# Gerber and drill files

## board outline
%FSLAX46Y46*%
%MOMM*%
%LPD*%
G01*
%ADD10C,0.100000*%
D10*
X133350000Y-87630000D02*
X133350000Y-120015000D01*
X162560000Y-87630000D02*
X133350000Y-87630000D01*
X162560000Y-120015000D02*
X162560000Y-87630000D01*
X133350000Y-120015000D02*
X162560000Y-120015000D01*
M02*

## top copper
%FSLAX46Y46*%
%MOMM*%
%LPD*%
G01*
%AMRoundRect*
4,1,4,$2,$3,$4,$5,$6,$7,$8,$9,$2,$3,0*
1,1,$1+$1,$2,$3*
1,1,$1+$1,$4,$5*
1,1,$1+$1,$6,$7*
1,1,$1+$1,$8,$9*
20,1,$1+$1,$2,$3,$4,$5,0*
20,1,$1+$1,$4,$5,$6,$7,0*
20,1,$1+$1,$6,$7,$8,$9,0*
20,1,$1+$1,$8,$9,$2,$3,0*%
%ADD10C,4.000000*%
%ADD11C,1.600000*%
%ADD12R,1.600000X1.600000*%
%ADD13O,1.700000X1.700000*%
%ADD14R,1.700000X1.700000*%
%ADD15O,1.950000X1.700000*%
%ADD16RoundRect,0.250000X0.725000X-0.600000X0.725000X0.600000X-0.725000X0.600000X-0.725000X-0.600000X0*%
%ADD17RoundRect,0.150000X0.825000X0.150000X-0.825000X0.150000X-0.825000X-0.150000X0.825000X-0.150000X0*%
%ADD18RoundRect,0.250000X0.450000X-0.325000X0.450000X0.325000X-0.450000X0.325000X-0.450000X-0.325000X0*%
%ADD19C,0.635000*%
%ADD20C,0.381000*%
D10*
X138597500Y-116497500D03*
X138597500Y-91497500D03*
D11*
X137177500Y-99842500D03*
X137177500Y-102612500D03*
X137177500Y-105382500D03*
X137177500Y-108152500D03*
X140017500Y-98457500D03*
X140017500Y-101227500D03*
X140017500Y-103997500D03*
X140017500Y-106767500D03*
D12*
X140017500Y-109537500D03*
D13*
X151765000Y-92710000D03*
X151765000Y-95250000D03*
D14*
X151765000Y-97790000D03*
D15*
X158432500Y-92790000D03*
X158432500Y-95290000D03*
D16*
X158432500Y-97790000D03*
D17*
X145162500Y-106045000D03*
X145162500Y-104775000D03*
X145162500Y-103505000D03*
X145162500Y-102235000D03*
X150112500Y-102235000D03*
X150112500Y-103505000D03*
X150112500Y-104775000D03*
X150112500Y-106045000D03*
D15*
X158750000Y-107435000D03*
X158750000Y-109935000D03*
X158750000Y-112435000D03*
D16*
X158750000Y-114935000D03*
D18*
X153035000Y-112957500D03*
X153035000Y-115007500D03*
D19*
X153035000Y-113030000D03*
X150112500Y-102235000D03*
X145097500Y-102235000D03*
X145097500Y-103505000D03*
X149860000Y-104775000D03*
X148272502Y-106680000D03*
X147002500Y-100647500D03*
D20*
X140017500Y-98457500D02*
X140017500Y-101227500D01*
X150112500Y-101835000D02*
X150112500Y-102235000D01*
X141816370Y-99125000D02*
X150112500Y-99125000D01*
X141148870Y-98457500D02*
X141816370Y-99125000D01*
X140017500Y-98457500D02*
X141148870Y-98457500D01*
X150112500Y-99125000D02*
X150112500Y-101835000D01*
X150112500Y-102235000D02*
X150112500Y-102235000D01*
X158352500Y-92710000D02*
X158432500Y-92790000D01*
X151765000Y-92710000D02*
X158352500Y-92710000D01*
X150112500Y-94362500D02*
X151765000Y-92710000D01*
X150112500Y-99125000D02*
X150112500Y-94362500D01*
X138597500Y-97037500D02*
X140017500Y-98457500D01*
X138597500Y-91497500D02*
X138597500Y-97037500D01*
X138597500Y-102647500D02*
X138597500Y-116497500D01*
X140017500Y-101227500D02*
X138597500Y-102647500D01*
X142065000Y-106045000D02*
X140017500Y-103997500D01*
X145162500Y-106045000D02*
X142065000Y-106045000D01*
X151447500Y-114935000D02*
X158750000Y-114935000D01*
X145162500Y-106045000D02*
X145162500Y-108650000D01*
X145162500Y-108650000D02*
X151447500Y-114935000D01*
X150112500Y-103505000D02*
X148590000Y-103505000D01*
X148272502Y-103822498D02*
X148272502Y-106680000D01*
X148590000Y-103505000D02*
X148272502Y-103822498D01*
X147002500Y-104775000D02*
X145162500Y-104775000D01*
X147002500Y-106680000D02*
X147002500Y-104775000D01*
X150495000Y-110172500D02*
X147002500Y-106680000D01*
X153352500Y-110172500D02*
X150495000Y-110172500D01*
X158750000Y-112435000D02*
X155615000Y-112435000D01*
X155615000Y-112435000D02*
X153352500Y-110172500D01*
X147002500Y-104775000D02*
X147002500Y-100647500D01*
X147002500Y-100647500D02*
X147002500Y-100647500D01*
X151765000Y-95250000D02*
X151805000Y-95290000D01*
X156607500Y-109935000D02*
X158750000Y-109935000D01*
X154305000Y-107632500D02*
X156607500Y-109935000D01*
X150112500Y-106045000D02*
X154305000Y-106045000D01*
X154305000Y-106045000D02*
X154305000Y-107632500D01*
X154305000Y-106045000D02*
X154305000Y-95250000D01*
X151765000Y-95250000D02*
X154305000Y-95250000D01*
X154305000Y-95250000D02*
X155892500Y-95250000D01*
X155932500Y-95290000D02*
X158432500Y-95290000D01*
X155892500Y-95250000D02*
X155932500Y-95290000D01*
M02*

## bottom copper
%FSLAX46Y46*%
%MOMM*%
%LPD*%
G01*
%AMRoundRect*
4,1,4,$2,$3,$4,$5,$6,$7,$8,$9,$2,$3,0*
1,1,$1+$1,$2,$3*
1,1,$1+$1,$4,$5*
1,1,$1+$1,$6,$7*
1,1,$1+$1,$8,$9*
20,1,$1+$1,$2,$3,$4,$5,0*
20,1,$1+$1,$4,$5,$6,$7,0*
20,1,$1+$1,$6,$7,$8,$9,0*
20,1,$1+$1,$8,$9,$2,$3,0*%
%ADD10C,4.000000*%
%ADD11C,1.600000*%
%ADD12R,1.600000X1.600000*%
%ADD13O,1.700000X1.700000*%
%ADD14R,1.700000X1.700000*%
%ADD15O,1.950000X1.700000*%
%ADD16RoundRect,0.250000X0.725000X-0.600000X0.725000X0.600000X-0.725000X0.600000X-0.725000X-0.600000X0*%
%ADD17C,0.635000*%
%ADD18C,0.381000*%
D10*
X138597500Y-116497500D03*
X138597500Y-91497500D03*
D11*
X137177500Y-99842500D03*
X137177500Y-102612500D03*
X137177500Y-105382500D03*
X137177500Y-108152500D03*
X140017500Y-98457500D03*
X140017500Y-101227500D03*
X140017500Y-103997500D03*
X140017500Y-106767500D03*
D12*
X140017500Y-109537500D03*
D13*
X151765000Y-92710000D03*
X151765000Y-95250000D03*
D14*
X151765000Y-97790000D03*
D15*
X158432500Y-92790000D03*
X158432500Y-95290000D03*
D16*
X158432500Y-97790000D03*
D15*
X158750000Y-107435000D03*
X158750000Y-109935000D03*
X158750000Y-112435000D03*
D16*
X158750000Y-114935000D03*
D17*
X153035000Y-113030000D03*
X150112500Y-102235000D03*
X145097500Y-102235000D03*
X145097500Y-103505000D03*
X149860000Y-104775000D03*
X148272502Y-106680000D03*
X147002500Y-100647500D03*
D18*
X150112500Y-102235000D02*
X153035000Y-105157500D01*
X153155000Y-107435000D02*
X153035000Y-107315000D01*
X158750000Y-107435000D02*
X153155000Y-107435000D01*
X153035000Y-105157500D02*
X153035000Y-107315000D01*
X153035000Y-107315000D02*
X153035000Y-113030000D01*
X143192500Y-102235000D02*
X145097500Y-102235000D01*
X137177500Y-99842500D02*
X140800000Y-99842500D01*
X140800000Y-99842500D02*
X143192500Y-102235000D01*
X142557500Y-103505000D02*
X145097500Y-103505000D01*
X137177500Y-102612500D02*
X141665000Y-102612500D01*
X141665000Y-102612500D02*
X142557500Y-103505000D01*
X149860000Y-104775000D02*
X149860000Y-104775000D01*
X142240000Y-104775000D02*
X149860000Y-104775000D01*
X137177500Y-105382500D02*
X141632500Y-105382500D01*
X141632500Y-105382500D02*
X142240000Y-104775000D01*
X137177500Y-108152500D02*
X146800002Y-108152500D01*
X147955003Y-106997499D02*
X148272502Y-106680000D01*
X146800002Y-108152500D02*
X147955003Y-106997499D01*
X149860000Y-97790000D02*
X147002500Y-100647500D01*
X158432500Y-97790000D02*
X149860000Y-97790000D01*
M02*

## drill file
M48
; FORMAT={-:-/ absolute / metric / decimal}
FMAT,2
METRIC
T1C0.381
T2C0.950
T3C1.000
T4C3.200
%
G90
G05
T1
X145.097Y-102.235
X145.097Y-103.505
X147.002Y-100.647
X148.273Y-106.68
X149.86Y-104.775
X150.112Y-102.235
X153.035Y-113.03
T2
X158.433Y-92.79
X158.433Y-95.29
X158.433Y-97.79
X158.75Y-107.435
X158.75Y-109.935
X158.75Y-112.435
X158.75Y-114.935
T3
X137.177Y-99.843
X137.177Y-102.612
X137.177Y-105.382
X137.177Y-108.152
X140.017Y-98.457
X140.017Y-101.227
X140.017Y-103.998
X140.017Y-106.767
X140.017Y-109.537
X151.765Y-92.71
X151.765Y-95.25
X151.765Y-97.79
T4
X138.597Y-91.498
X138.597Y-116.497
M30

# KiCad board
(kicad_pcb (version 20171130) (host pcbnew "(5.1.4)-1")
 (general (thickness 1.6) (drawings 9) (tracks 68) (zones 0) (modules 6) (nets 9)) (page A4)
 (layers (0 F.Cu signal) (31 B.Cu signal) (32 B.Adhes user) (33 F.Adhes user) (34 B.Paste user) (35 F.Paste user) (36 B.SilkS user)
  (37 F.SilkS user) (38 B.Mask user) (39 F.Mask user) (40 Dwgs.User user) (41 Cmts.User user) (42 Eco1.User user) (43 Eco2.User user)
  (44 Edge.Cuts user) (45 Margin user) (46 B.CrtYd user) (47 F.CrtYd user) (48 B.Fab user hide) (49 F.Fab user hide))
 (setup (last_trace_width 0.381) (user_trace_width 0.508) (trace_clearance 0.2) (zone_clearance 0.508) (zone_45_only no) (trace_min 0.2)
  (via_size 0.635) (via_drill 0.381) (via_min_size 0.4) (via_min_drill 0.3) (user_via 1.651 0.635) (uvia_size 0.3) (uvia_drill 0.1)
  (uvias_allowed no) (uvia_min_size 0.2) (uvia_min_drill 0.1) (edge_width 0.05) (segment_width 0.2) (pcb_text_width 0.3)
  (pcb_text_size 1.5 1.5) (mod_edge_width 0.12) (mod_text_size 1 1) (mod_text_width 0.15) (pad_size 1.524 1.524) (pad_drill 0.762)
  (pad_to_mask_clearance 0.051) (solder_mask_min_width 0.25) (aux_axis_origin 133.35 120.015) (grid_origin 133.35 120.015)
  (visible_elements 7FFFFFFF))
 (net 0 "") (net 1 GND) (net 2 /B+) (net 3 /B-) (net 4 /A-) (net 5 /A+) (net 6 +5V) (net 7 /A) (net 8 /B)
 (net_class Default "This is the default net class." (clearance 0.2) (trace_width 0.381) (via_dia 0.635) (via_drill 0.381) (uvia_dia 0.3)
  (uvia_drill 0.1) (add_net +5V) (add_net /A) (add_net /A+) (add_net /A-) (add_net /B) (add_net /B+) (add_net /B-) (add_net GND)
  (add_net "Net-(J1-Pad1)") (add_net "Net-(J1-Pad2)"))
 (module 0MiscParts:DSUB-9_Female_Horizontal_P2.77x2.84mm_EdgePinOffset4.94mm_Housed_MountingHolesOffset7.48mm (layer F.Cu)
  (at 140.0175 109.5375 270)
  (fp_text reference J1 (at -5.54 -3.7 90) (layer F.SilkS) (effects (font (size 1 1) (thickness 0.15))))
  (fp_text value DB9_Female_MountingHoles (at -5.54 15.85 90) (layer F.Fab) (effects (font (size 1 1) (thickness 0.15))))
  (pad 0 thru_hole circle (at 6.96 1.42 270) (size 4 4) (drill 3.2) (layers *.Cu *.Mask) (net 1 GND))
  (pad 0 thru_hole circle (at -18.04 1.42 270) (size 4 4) (drill 3.2) (layers *.Cu *.Mask) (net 1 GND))
  (pad 9 thru_hole circle (at -9.695 2.84 270) (size 1.6 1.6) (drill 1) (layers *.Cu *.Mask) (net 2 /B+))
  (pad 8 thru_hole circle (at -6.925 2.84 270) (size 1.6 1.6) (drill 1) (layers *.Cu *.Mask) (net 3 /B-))
  (pad 7 thru_hole circle (at -4.155 2.84 270) (size 1.6 1.6) (drill 1) (layers *.Cu *.Mask) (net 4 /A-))
  (pad 6 thru_hole circle (at -1.385 2.84 270) (size 1.6 1.6) (drill 1) (layers *.Cu *.Mask) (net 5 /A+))
  (pad 5 thru_hole circle (at -11.08 0 270) (size 1.6 1.6) (drill 1) (layers *.Cu *.Mask) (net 1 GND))
  (pad 4 thru_hole circle (at -8.31 0 270) (size 1.6 1.6) (drill 1) (layers *.Cu *.Mask) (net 1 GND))
  (pad 3 thru_hole circle (at -5.54 0 270) (size 1.6 1.6) (drill 1) (layers *.Cu *.Mask) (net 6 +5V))
  (pad 2 thru_hole circle (at -2.77 0 270) (size 1.6 1.6) (drill 1) (layers *.Cu *.Mask))
  (pad 1 thru_hole rect (at 0 0 270) (size 1.6 1.6) (drill 1) (layers *.Cu *.Mask)))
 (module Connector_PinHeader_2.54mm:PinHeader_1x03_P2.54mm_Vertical (layer F.Cu) (at 151.765 97.79 180)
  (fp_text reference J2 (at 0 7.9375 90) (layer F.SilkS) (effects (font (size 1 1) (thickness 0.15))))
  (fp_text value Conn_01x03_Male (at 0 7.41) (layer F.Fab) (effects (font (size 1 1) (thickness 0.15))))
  (pad 3 thru_hole oval (at 0 5.08 180) (size 1.7 1.7) (drill 1) (layers *.Cu *.Mask) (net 1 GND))
  (pad 2 thru_hole oval (at 0 2.54 180) (size 1.7 1.7) (drill 1) (layers *.Cu *.Mask) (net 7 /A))
  (pad 1 thru_hole rect (at 0 0 180) (size 1.7 1.7) (drill 1) (layers *.Cu *.Mask) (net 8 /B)))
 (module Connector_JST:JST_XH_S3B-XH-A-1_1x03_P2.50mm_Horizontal (layer F.Cu) (at 158.4325 97.79 90)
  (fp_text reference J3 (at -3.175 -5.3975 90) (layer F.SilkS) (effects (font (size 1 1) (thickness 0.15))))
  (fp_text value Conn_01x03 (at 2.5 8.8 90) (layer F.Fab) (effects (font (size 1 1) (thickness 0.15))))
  (pad 3 thru_hole oval (at 5 0 90) (size 1.7 1.95) (drill 0.95) (layers *.Cu *.Mask) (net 1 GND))
  (pad 2 thru_hole oval (at 2.5 0 90) (size 1.7 1.95) (drill 0.95) (layers *.Cu *.Mask) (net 7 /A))
  (pad 1 thru_hole roundrect (at 0 0 90) (size 1.7 1.95) (drill 0.95) (layers *.Cu *.Mask) (roundrect_rratio 0.147059) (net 8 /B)))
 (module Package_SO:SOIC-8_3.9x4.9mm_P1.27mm (layer F.Cu) (at 147.6375 104.14 180)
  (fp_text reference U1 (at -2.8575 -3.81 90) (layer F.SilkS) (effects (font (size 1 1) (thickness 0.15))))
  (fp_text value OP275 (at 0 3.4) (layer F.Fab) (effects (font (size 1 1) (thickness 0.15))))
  (pad 8 smd roundrect (at 2.475 -1.905 180) (size 1.95 0.6) (layers F.Cu F.Paste F.Mask) (roundrect_rratio 0.25) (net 6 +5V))
  (pad 7 smd roundrect (at 2.475 -0.635 180) (size 1.95 0.6) (layers F.Cu F.Paste F.Mask) (roundrect_rratio 0.25) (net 8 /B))
  (pad 6 smd roundrect (at 2.475 0.635 180) (size 1.95 0.6) (layers F.Cu F.Paste F.Mask) (roundrect_rratio 0.25) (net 3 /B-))
  (pad 5 smd roundrect (at 2.475 1.905 180) (size 1.95 0.6) (layers F.Cu F.Paste F.Mask) (roundrect_rratio 0.25) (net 2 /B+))
  (pad 4 smd roundrect (at -2.475 1.905 180) (size 1.95 0.6) (layers F.Cu F.Paste F.Mask) (roundrect_rratio 0.25) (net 1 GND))
  (pad 3 smd roundrect (at -2.475 0.635 180) (size 1.95 0.6) (layers F.Cu F.Paste F.Mask) (roundrect_rratio 0.25) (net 5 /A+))
  (pad 2 smd roundrect (at -2.475 -0.635 180) (size 1.95 0.6) (layers F.Cu F.Paste F.Mask) (roundrect_rratio 0.25) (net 4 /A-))
  (pad 1 smd roundrect (at -2.475 -1.905 180) (size 1.95 0.6) (layers F.Cu F.Paste F.Mask) (roundrect_rratio 0.25) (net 7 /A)))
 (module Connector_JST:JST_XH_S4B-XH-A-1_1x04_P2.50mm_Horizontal (layer F.Cu) (at 158.75 114.935 90)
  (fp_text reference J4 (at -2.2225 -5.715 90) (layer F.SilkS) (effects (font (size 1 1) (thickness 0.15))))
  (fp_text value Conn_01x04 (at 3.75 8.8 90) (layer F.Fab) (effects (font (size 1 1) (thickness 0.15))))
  (pad 4 thru_hole oval (at 7.5 0 90) (size 1.7 1.95) (drill 0.95) (layers *.Cu *.Mask) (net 1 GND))
  (pad 3 thru_hole oval (at 5 0 90) (size 1.7 1.95) (drill 0.95) (layers *.Cu *.Mask) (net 7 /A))
  (pad 2 thru_hole oval (at 2.5 0 90) (size 1.7 1.95) (drill 0.95) (layers *.Cu *.Mask) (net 8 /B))
  (pad 1 thru_hole roundrect (at 0 0 90) (size 1.7 1.95) (drill 0.95) (layers *.Cu *.Mask) (roundrect_rratio 0.147059) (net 6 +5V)))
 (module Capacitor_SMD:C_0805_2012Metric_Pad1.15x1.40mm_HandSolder (layer F.Cu) (at 153.035 113.9825 90)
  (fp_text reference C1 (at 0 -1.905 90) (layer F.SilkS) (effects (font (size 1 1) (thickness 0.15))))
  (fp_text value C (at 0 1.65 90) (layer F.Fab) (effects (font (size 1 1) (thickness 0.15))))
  (pad 2 smd roundrect (at 1.025 0 90) (size 1.15 1.4) (layers F.Cu F.Paste F.Mask) (roundrect_rratio 0.217391) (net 1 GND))
  (pad 1 smd roundrect (at -1.025 0 90) (size 1.15 1.4) (layers F.Cu F.Paste F.Mask) (roundrect_rratio 0.217391) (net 6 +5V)))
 (gr_line (start 133.35 87.63) (end 133.35 120.015) (layer Edge.Cuts) (width 0.1))
 (gr_line (start 162.56 87.63) (end 133.35 87.63) (layer Edge.Cuts) (width 0.1))
 (gr_line (start 162.56 120.015) (end 162.56 87.63) (layer Edge.Cuts) (width 0.1))
 (gr_line (start 133.35 120.015) (end 162.56 120.015) (layer Edge.Cuts) (width 0.1))
 (via (at 153.035 113.03) (size 0.635) (drill 0.381) (layers F.Cu B.Cu) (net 1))
 (segment (start 140.0175 98.4575) (end 140.0175 101.2275) (width 0.381) (layer F.Cu) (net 1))
 (segment (start 150.1125 101.835) (end 150.1125 102.235) (width 0.381) (layer F.Cu) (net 1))
 (segment (start 141.81637 99.125) (end 150.1125 99.125) (width 0.381) (layer F.Cu) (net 1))
 (segment (start 141.14887 98.4575) (end 141.81637 99.125) (width 0.381) (layer F.Cu) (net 1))
 (segment (start 140.0175 98.4575) (end 141.14887 98.4575) (width 0.381) (layer F.Cu) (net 1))
 (segment (start 150.1125 99.125) (end 150.1125 101.835) (width 0.381) (layer F.Cu) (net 1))
 (segment (start 150.1125 102.235) (end 150.1125 102.235) (width 0.381) (layer F.Cu) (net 1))
 (via (at 150.1125 102.235) (size 0.635) (drill 0.381) (layers F.Cu B.Cu) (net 1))
 (segment (start 150.1125 102.235) (end 153.035 105.1575) (width 0.381) (layer B.Cu) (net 1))
 (segment (start 153.155 107.435) (end 153.035 107.315) (width 0.381) (layer B.Cu) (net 1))
 (segment (start 158.75 107.435) (end 153.155 107.435) (width 0.381) (layer B.Cu) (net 1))
 (segment (start 153.035 105.1575) (end 153.035 107.315) (width 0.381) (layer B.Cu) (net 1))
 (segment (start 153.035 107.315) (end 153.035 113.03) (width 0.381) (layer B.Cu) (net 1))
 (segment (start 158.3525 92.71) (end 158.4325 92.79) (width 0.381) (layer F.Cu) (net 1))
 (segment (start 151.765 92.71) (end 158.3525 92.71) (width 0.381) (layer F.Cu) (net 1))
 (segment (start 150.1125 94.3625) (end 151.765 92.71) (width 0.381) (layer F.Cu) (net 1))
 (segment (start 150.1125 99.125) (end 150.1125 94.3625) (width 0.381) (layer F.Cu) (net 1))
 (segment (start 138.5975 97.0375) (end 140.0175 98.4575) (width 0.381) (layer F.Cu) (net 1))
 (segment (start 138.5975 91.4975) (end 138.5975 97.0375) (width 0.381) (layer F.Cu) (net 1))
 (segment (start 138.5975 102.6475) (end 138.5975 116.4975) (width 0.381) (layer F.Cu) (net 1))
 (segment (start 140.0175 101.2275) (end 138.5975 102.6475) (width 0.381) (layer F.Cu) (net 1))
 (segment (start 142.065 106.045) (end 140.0175 103.9975) (width 0.381) (layer F.Cu) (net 6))
 (segment (start 145.1625 106.045) (end 142.065 106.045) (width 0.381) (layer F.Cu) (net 6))
 (segment (start 151.4475 114.935) (end 158.75 114.935) (width 0.381) (layer F.Cu) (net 6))
 (segment (start 145.1625 106.045) (end 145.1625 108.65) (width 0.381) (layer F.Cu) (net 6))
 (segment (start 145.1625 108.65) (end 151.4475 114.935) (width 0.381) (layer F.Cu) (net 6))
 (via (at 145.0975 102.235) (size 0.635) (drill 0.381) (layers F.Cu B.Cu) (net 2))
 (segment (start 143.1925 102.235) (end 145.0975 102.235) (width 0.381) (layer B.Cu) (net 2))
 (segment (start 137.1775 99.8425) (end 140.8 99.8425) (width 0.381) (layer B.Cu) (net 2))
 (segment (start 140.8 99.8425) (end 143.1925 102.235) (width 0.381) (layer B.Cu) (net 2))
 (via (at 145.0975 103.505) (size 0.635) (drill 0.381) (layers F.Cu B.Cu) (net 3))
 (segment (start 142.5575 103.505) (end 145.0975 103.505) (width 0.381) (layer B.Cu) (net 3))
 (segment (start 137.1775 102.6125) (end 141.665 102.6125) (width 0.381) (layer B.Cu) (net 3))
 (segment (start 141.665 102.6125) (end 142.5575 103.505) (width 0.381) (layer B.Cu) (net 3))
 (segment (start 149.86 104.775) (end 149.86 104.775) (width 0.381) (layer B.Cu) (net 4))
 (via (at 149.86 104.775) (size 0.635) (drill 0.381) (layers F.Cu B.Cu) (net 4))
 (segment (start 142.24 104.775) (end 149.86 104.775) (width 0.381) (layer B.Cu) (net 4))
 (segment (start 137.1775 105.3825) (end 141.6325 105.3825) (width 0.381) (layer B.Cu) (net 4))
 (segment (start 141.6325 105.3825) (end 142.24 104.775) (width 0.381) (layer B.Cu) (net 4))
 (via (at 148.272502 106.68) (size 0.635) (drill 0.381) (layers F.Cu B.Cu) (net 5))
 (segment (start 137.1775 108.1525) (end 146.800002 108.1525) (width 0.381) (layer B.Cu) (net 5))
 (segment (start 147.955003 106.997499) (end 148.272502 106.68) (width 0.381) (layer B.Cu) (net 5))
 (segment (start 146.800002 108.1525) (end 147.955003 106.997499) (width 0.381) (layer B.Cu) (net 5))
 (segment (start 150.1125 103.505) (end 148.59 103.505) (width 0.381) (layer F.Cu) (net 5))
 (segment (start 148.272502 103.822498) (end 148.272502 106.68) (width 0.381) (layer F.Cu) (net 5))
 (segment (start 148.59 103.505) (end 148.272502 103.822498) (width 0.381) (layer F.Cu) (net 5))
 (segment (start 147.0025 104.775) (end 145.1625 104.775) (width 0.381) (layer F.Cu) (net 8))
 (segment (start 147.0025 106.68) (end 147.0025 104.775) (width 0.381) (layer F.Cu) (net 8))
 (segment (start 150.495 110.1725) (end 147.0025 106.68) (width 0.381) (layer F.Cu) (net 8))
 (segment (start 153.3525 110.1725) (end 150.495 110.1725) (width 0.381) (layer F.Cu) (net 8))
 (segment (start 158.75 112.435) (end 155.615 112.435) (width 0.381) (layer F.Cu) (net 8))
 (segment (start 155.615 112.435) (end 153.3525 110.1725) (width 0.381) (layer F.Cu) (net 8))
 (segment (start 147.0025 104.775) (end 147.0025 100.6475) (width 0.381) (layer F.Cu) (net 8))
 (segment (start 147.0025 100.6475) (end 147.0025 100.6475) (width 0.381) (layer F.Cu) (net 8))
 (via (at 147.0025 100.6475) (size 0.635) (drill 0.381) (layers F.Cu B.Cu) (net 8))
 (segment (start 149.86 97.79) (end 147.0025 100.6475) (width 0.381) (layer B.Cu) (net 8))
 (segment (start 158.4325 97.79) (end 149.86 97.79) (width 0.381) (layer B.Cu) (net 8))
 (segment (start 151.765 95.25) (end 151.805 95.29) (width 0.381) (layer F.Cu) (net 7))
 (segment (start 156.6075 109.935) (end 158.75 109.935) (width 0.381) (layer F.Cu) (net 7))
 (segment (start 154.305 107.6325) (end 156.6075 109.935) (width 0.381) (layer F.Cu) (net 7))
 (segment (start 150.1125 106.045) (end 154.305 106.045) (width 0.381) (layer F.Cu) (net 7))
 (segment (start 154.305 106.045) (end 154.305 107.6325) (width 0.381) (layer F.Cu) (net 7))
 (segment (start 154.305 106.045) (end 154.305 95.25) (width 0.381) (layer F.Cu) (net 7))
 (segment (start 151.765 95.25) (end 154.305 95.25) (width 0.381) (layer F.Cu) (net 7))
 (segment (start 154.305 95.25) (end 155.8925 95.25) (width 0.381) (layer F.Cu) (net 7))
 (segment (start 155.9325 95.29) (end 158.4325 95.29) (width 0.381) (layer F.Cu) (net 7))
 (segment (start 155.8925 95.25) (end 155.9325 95.29) (width 0.381) (layer F.Cu) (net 7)))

